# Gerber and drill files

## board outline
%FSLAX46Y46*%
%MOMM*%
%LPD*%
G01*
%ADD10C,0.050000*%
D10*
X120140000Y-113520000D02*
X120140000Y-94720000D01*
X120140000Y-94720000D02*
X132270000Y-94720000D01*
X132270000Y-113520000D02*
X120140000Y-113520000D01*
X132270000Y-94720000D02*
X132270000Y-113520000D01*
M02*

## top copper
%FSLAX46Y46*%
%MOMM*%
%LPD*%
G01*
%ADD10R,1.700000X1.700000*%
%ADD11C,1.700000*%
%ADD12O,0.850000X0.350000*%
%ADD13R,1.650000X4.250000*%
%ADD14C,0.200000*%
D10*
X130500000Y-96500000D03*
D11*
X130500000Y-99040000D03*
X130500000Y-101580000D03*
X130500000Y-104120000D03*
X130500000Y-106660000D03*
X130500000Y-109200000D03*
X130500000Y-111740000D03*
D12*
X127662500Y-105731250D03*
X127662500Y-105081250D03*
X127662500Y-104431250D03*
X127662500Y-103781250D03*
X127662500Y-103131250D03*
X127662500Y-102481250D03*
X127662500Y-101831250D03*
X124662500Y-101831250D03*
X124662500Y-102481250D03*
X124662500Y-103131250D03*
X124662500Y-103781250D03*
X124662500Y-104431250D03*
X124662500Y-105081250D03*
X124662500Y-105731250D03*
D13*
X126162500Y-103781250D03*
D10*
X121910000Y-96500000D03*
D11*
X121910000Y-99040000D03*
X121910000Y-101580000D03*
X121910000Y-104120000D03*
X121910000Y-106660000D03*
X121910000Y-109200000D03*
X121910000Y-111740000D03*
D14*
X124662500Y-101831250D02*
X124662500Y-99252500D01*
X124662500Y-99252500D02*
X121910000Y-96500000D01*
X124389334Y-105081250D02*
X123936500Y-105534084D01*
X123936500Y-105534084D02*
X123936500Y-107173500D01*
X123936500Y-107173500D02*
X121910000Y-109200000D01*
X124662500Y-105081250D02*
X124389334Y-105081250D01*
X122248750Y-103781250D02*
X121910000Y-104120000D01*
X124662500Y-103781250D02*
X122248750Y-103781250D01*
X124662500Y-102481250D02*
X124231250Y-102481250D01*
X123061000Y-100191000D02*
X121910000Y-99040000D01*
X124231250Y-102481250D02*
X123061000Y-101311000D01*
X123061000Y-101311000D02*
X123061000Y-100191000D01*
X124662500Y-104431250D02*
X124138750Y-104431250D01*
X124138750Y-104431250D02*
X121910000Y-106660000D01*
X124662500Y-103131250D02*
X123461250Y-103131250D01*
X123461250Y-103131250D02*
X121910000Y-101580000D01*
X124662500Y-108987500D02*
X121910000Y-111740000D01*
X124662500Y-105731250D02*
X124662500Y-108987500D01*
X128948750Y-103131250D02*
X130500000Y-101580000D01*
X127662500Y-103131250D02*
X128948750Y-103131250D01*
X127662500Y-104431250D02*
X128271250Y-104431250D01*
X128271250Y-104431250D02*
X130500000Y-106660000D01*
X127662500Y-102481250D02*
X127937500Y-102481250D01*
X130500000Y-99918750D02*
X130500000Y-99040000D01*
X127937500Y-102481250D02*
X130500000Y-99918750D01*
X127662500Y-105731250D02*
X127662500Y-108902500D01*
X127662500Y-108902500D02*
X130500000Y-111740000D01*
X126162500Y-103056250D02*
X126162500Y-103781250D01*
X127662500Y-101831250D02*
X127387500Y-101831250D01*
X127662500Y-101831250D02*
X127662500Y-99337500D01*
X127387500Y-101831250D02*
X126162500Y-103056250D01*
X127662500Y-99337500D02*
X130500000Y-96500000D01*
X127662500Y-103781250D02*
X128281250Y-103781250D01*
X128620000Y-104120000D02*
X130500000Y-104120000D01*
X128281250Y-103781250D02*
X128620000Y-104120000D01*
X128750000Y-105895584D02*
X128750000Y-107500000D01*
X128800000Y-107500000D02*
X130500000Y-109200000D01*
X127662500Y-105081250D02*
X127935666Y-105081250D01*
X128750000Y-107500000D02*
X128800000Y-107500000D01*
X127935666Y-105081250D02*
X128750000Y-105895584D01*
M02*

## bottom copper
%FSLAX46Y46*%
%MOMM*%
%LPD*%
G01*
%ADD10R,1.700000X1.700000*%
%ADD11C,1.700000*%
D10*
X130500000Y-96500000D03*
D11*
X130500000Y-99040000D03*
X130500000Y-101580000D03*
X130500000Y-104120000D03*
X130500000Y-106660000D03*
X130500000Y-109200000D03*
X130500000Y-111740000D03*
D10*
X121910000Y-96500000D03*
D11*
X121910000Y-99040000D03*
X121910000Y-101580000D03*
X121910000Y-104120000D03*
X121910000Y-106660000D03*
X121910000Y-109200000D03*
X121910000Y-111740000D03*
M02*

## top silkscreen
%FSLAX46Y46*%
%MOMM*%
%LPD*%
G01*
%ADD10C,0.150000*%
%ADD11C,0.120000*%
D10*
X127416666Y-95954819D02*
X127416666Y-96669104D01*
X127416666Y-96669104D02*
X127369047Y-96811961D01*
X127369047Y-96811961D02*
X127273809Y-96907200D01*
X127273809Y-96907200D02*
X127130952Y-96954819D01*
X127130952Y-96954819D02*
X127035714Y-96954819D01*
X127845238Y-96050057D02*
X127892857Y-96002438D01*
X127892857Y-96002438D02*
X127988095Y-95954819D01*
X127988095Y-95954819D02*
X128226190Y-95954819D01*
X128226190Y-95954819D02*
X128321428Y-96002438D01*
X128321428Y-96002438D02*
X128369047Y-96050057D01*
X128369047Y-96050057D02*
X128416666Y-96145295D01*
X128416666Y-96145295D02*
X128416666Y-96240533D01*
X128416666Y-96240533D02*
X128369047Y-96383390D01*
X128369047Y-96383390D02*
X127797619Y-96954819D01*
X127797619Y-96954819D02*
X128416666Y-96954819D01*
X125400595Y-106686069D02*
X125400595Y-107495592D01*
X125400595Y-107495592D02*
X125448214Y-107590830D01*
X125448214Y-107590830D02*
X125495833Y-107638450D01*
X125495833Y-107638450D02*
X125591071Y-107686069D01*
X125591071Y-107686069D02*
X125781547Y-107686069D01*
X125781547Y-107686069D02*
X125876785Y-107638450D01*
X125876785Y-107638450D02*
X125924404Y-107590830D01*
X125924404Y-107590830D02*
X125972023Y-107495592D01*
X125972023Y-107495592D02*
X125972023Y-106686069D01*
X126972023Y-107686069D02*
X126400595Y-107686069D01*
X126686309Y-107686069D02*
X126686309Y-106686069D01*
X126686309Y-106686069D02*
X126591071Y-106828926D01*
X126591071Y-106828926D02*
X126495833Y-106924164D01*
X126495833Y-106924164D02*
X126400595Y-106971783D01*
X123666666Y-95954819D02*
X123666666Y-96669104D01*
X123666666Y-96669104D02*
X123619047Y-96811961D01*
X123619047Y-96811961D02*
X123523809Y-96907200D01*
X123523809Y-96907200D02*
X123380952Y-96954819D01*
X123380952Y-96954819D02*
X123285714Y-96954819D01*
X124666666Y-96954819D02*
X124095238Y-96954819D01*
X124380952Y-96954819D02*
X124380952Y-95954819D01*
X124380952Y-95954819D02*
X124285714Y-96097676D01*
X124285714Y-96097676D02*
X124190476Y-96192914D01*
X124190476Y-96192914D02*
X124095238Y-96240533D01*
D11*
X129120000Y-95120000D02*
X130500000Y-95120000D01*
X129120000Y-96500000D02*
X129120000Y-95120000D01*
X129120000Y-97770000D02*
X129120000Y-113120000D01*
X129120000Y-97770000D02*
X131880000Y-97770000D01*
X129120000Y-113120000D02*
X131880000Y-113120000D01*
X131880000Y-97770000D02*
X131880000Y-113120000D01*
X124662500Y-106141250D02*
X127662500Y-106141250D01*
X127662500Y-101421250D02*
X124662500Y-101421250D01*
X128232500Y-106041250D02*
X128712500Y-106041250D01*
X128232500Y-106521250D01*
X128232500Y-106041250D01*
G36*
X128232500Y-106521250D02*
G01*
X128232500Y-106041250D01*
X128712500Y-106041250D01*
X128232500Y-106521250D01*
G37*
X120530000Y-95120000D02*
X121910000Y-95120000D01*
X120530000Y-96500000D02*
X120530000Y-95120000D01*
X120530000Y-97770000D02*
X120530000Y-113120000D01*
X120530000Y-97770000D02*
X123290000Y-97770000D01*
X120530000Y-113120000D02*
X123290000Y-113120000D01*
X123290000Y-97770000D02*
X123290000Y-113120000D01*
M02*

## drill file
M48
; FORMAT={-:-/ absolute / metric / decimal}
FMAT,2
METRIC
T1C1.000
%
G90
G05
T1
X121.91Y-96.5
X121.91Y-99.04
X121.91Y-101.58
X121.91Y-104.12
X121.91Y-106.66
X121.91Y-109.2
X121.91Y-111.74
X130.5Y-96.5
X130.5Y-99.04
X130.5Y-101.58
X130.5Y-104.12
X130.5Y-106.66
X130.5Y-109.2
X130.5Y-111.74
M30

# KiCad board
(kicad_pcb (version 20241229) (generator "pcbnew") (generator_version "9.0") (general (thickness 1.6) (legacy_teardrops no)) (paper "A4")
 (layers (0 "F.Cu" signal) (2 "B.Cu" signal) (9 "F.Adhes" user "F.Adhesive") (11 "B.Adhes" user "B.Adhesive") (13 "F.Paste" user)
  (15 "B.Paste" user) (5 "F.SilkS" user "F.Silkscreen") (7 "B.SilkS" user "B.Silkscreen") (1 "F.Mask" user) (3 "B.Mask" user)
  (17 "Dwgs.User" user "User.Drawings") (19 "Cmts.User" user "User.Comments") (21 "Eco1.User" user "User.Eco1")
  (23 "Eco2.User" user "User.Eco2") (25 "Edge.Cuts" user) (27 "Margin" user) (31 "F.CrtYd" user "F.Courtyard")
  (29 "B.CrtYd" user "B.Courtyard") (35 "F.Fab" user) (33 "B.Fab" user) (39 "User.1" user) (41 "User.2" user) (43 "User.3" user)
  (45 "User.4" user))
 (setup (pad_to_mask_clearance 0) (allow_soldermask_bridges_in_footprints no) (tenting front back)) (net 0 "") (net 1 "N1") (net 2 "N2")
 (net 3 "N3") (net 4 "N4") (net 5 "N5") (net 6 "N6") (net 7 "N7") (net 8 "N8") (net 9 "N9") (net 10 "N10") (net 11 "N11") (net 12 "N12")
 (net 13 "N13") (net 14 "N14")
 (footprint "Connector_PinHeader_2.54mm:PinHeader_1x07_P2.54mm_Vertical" (layer "F.Cu") (at 130.5 96.5)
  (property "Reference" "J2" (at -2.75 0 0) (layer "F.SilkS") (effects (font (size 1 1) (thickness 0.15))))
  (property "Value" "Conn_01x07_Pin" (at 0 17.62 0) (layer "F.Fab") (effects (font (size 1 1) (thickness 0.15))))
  (fp_line (start -1.38 -1.38) (end 0 -1.38) (stroke (width 0.12) (type solid)) (layer "F.SilkS"))
  (fp_line (start -1.38 0) (end -1.38 -1.38) (stroke (width 0.12) (type solid)) (layer "F.SilkS"))
  (fp_line (start -1.38 1.27) (end -1.38 16.62) (stroke (width 0.12) (type solid)) (layer "F.SilkS"))
  (fp_line (start -1.38 1.27) (end 1.38 1.27) (stroke (width 0.12) (type solid)) (layer "F.SilkS"))
  (fp_line (start -1.38 16.62) (end 1.38 16.62) (stroke (width 0.12) (type solid)) (layer "F.SilkS"))
  (fp_line (start 1.38 1.27) (end 1.38 16.62) (stroke (width 0.12) (type solid)) (layer "F.SilkS"))
  (pad "1" thru_hole rect (at 0 0) (size 1.7 1.7) (drill 1) (layers "*.Cu" "*.Mask") (remove_unused_layers no) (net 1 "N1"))
  (pad "2" thru_hole circle (at 0 2.54) (size 1.7 1.7) (drill 1) (layers "*.Cu" "*.Mask") (remove_unused_layers no) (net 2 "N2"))
  (pad "3" thru_hole circle (at 0 5.08) (size 1.7 1.7) (drill 1) (layers "*.Cu" "*.Mask") (remove_unused_layers no) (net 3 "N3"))
  (pad "4" thru_hole circle (at 0 7.62) (size 1.7 1.7) (drill 1) (layers "*.Cu" "*.Mask") (remove_unused_layers no) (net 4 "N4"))
  (pad "5" thru_hole circle (at 0 10.16) (size 1.7 1.7) (drill 1) (layers "*.Cu" "*.Mask") (remove_unused_layers no) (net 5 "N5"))
  (pad "6" thru_hole circle (at 0 12.7) (size 1.7 1.7) (drill 1) (layers "*.Cu" "*.Mask") (remove_unused_layers no) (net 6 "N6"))
  (pad "7" thru_hole circle (at 0 15.24) (size 1.7 1.7) (drill 1) (layers "*.Cu" "*.Mask") (remove_unused_layers no) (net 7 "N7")))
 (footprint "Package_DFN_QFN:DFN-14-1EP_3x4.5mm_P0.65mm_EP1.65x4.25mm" (layer "F.Cu") (at 126.1625 103.78125 180)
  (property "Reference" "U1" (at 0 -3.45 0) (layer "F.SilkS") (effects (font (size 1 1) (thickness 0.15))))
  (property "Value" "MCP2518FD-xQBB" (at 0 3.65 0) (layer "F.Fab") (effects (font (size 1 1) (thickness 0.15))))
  (fp_line (start 1.5 -2.36) (end -1.5 -2.36) (stroke (width 0.12) (type solid)) (layer "F.SilkS"))
  (fp_line (start -1.5 2.36) (end 1.5 2.36) (stroke (width 0.12) (type solid)) (layer "F.SilkS"))
  (fp_poly
   (pts (xy -2.07 -2.26) (xy -2.55 -2.26) (xy -2.07 -2.74) (xy -2.07 -2.26)) (stroke (width 0.12) (type solid)) (fill yes) (layer "F.SilkS"))
  (pad "" smd rect (at -0.4125 -1.59375 180) (size 0.66 0.85) (layers "F.Paste"))
  (pad "" smd rect (at -0.4125 -0.53125 180) (size 0.66 0.85) (layers "F.Paste"))
  (pad "" smd rect (at -0.4125 0.53125 180) (size 0.66 0.85) (layers "F.Paste"))
  (pad "" smd rect (at -0.4125 1.59375 180) (size 0.66 0.85) (layers "F.Paste"))
  (pad "" smd rect (at 0.4125 -1.59375 180) (size 0.66 0.85) (layers "F.Paste"))
  (pad "" smd rect (at 0.4125 -0.53125 180) (size 0.66 0.85) (layers "F.Paste"))
  (pad "" smd rect (at 0.4125 0.53125 180) (size 0.66 0.85) (layers "F.Paste"))
  (pad "" smd rect (at 0.4125 1.59375 180) (size 0.66 0.85) (layers "F.Paste"))
  (pad "1" smd oval (at -1.5 -1.95 180) (size 0.85 0.35) (layers "F.Cu" "F.Mask" "F.Paste") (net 7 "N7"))
  (pad "2" smd oval (at -1.5 -1.3 180) (size 0.85 0.35) (layers "F.Cu" "F.Mask" "F.Paste") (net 6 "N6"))
  (pad "3" smd oval (at -1.5 -0.65 180) (size 0.85 0.35) (layers "F.Cu" "F.Mask" "F.Paste") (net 5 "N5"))
  (pad "4" smd oval (at -1.5 0 180) (size 0.85 0.35) (layers "F.Cu" "F.Mask" "F.Paste") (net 4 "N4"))
  (pad "5" smd oval (at -1.5 0.65 180) (size 0.85 0.35) (layers "F.Cu" "F.Mask" "F.Paste") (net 3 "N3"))
  (pad "6" smd oval (at -1.5 1.3 180) (size 0.85 0.35) (layers "F.Cu" "F.Mask" "F.Paste") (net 2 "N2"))
  (pad "7" smd oval (at -1.5 1.95 180) (size 0.85 0.35) (layers "F.Cu" "F.Mask" "F.Paste") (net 1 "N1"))
  (pad "8" smd oval (at 1.5 1.95 180) (size 0.85 0.35) (layers "F.Cu" "F.Mask" "F.Paste") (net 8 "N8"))
  (pad "9" smd oval (at 1.5 1.3 180) (size 0.85 0.35) (layers "F.Cu" "F.Mask" "F.Paste") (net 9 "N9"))
  (pad "10" smd oval (at 1.5 0.65 180) (size 0.85 0.35) (layers "F.Cu" "F.Mask" "F.Paste") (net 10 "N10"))
  (pad "11" smd oval (at 1.5 0 180) (size 0.85 0.35) (layers "F.Cu" "F.Mask" "F.Paste") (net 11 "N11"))
  (pad "12" smd oval (at 1.5 -0.65 180) (size 0.85 0.35) (layers "F.Cu" "F.Mask" "F.Paste") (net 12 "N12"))
  (pad "13" smd oval (at 1.5 -1.3 180) (size 0.85 0.35) (layers "F.Cu" "F.Mask" "F.Paste") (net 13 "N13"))
  (pad "14" smd oval (at 1.5 -1.95 180) (size 0.85 0.35) (layers "F.Cu" "F.Mask" "F.Paste") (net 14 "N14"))
  (pad "15" smd rect (at 0 0 180) (size 1.65 4.25) (layers "F.Cu" "F.Mask") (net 1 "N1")))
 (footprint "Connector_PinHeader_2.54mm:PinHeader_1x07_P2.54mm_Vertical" (layer "F.Cu") (at 121.91 96.5)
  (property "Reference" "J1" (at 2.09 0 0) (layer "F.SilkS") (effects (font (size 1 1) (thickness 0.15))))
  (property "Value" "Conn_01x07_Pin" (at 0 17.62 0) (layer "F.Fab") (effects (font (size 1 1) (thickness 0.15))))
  (fp_line (start -1.38 -1.38) (end 0 -1.38) (stroke (width 0.12) (type solid)) (layer "F.SilkS"))
  (fp_line (start -1.38 0) (end -1.38 -1.38) (stroke (width 0.12) (type solid)) (layer "F.SilkS"))
  (fp_line (start -1.38 1.27) (end -1.38 16.62) (stroke (width 0.12) (type solid)) (layer "F.SilkS"))
  (fp_line (start -1.38 1.27) (end 1.38 1.27) (stroke (width 0.12) (type solid)) (layer "F.SilkS"))
  (fp_line (start -1.38 16.62) (end 1.38 16.62) (stroke (width 0.12) (type solid)) (layer "F.SilkS"))
  (fp_line (start 1.38 1.27) (end 1.38 16.62) (stroke (width 0.12) (type solid)) (layer "F.SilkS"))
  (pad "1" thru_hole rect (at 0 0) (size 1.7 1.7) (drill 1) (layers "*.Cu" "*.Mask") (remove_unused_layers no) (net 8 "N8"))
  (pad "2" thru_hole circle (at 0 2.54) (size 1.7 1.7) (drill 1) (layers "*.Cu" "*.Mask") (remove_unused_layers no) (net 9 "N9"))
  (pad "3" thru_hole circle (at 0 5.08) (size 1.7 1.7) (drill 1) (layers "*.Cu" "*.Mask") (remove_unused_layers no) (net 10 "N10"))
  (pad "4" thru_hole circle (at 0 7.62) (size 1.7 1.7) (drill 1) (layers "*.Cu" "*.Mask") (remove_unused_layers no) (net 11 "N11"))
  (pad "5" thru_hole circle (at 0 10.16) (size 1.7 1.7) (drill 1) (layers "*.Cu" "*.Mask") (remove_unused_layers no) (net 12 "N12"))
  (pad "6" thru_hole circle (at 0 12.7) (size 1.7 1.7) (drill 1) (layers "*.Cu" "*.Mask") (remove_unused_layers no) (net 13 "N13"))
  (pad "7" thru_hole circle (at 0 15.24) (size 1.7 1.7) (drill 1) (layers "*.Cu" "*.Mask") (remove_unused_layers no) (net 14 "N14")))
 (gr_line (start 120.14 113.52) (end 120.14 94.72) (stroke (width 0.05) (type default)) (layer "Edge.Cuts"))
 (gr_line (start 120.14 94.72) (end 132.27 94.72) (stroke (width 0.05) (type default)) (layer "Edge.Cuts"))
 (gr_line (start 132.27 113.52) (end 120.14 113.52) (stroke (width 0.05) (type default)) (layer "Edge.Cuts"))
 (gr_line (start 132.27 94.72) (end 132.27 113.52) (stroke (width 0.05) (type default)) (layer "Edge.Cuts"))
 (segment (start 124.6625 101.83125) (end 124.6625 99.2525) (width 0.2) (layer "F.Cu") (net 8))
 (segment (start 124.6625 99.2525) (end 121.91 96.5) (width 0.2) (layer "F.Cu") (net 8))
 (segment (start 124.389334 105.08125) (end 123.9365 105.534084) (width 0.2) (layer "F.Cu") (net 13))
 (segment (start 123.9365 105.534084) (end 123.9365 107.1735) (width 0.2) (layer "F.Cu") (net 13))
 (segment (start 123.9365 107.1735) (end 121.91 109.2) (width 0.2) (layer "F.Cu") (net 13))
 (segment (start 124.6625 105.08125) (end 124.389334 105.08125) (width 0.2) (layer "F.Cu") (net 13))
 (segment (start 122.24875 103.78125) (end 121.91 104.12) (width 0.2) (layer "F.Cu") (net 11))
 (segment (start 124.6625 103.78125) (end 122.24875 103.78125) (width 0.2) (layer "F.Cu") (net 11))
 (segment (start 124.6625 102.48125) (end 124.23125 102.48125) (width 0.2) (layer "F.Cu") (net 9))
 (segment (start 123.061 100.191) (end 121.91 99.04) (width 0.2) (layer "F.Cu") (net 9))
 (segment (start 124.23125 102.48125) (end 123.061 101.311) (width 0.2) (layer "F.Cu") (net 9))
 (segment (start 123.061 101.311) (end 123.061 100.191) (width 0.2) (layer "F.Cu") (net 9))
 (segment (start 124.6625 104.43125) (end 124.13875 104.43125) (width 0.2) (layer "F.Cu") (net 12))
 (segment (start 124.13875 104.43125) (end 121.91 106.66) (width 0.2) (layer "F.Cu") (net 12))
 (segment (start 124.6625 103.13125) (end 123.46125 103.13125) (width 0.2) (layer "F.Cu") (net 10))
 (segment (start 123.46125 103.13125) (end 121.91 101.58) (width 0.2) (layer "F.Cu") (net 10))
 (segment (start 124.6625 108.9875) (end 121.91 111.74) (width 0.2) (layer "F.Cu") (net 14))
 (segment (start 124.6625 105.73125) (end 124.6625 108.9875) (width 0.2) (layer "F.Cu") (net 14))
 (segment (start 128.94875 103.13125) (end 130.5 101.58) (width 0.2) (layer "F.Cu") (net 3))
 (segment (start 127.6625 103.13125) (end 128.94875 103.13125) (width 0.2) (layer "F.Cu") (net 3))
 (segment (start 127.6625 104.43125) (end 128.27125 104.43125) (width 0.2) (layer "F.Cu") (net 5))
 (segment (start 128.27125 104.43125) (end 130.5 106.66) (width 0.2) (layer "F.Cu") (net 5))
 (segment (start 127.6625 102.48125) (end 127.9375 102.48125) (width 0.2) (layer "F.Cu") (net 2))
 (segment (start 130.5 99.91875) (end 130.5 99.04) (width 0.2) (layer "F.Cu") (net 2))
 (segment (start 127.9375 102.48125) (end 130.5 99.91875) (width 0.2) (layer "F.Cu") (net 2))
 (segment (start 127.6625 105.73125) (end 127.6625 108.9025) (width 0.2) (layer "F.Cu") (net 7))
 (segment (start 127.6625 108.9025) (end 130.5 111.74) (width 0.2) (layer "F.Cu") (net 7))
 (segment (start 126.1625 103.05625) (end 126.1625 103.78125) (width 0.2) (layer "F.Cu") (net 1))
 (segment (start 127.6625 101.83125) (end 127.3875 101.83125) (width 0.2) (layer "F.Cu") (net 1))
 (segment (start 127.6625 101.83125) (end 127.6625 99.3375) (width 0.2) (layer "F.Cu") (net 1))
 (segment (start 127.3875 101.83125) (end 126.1625 103.05625) (width 0.2) (layer "F.Cu") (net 1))
 (segment (start 127.6625 99.3375) (end 130.5 96.5) (width 0.2) (layer "F.Cu") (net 1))
 (segment (start 127.6625 103.78125) (end 128.28125 103.78125) (width 0.2) (layer "F.Cu") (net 4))
 (segment (start 128.62 104.12) (end 130.5 104.12) (width 0.2) (layer "F.Cu") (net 4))
 (segment (start 128.28125 103.78125) (end 128.62 104.12) (width 0.2) (layer "F.Cu") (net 4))
 (segment (start 128.75 105.895584) (end 128.75 107.5) (width 0.2) (layer "F.Cu") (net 6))
 (segment (start 128.8 107.5) (end 130.5 109.2) (width 0.2) (layer "F.Cu") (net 6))
 (segment (start 127.6625 105.08125) (end 127.935666 105.08125) (width 0.2) (layer "F.Cu") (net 6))
 (segment (start 128.75 107.5) (end 128.8 107.5) (width 0.2) (layer "F.Cu") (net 6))
 (segment (start 127.935666 105.08125) (end 128.75 105.895584) (width 0.2) (layer "F.Cu") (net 6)))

